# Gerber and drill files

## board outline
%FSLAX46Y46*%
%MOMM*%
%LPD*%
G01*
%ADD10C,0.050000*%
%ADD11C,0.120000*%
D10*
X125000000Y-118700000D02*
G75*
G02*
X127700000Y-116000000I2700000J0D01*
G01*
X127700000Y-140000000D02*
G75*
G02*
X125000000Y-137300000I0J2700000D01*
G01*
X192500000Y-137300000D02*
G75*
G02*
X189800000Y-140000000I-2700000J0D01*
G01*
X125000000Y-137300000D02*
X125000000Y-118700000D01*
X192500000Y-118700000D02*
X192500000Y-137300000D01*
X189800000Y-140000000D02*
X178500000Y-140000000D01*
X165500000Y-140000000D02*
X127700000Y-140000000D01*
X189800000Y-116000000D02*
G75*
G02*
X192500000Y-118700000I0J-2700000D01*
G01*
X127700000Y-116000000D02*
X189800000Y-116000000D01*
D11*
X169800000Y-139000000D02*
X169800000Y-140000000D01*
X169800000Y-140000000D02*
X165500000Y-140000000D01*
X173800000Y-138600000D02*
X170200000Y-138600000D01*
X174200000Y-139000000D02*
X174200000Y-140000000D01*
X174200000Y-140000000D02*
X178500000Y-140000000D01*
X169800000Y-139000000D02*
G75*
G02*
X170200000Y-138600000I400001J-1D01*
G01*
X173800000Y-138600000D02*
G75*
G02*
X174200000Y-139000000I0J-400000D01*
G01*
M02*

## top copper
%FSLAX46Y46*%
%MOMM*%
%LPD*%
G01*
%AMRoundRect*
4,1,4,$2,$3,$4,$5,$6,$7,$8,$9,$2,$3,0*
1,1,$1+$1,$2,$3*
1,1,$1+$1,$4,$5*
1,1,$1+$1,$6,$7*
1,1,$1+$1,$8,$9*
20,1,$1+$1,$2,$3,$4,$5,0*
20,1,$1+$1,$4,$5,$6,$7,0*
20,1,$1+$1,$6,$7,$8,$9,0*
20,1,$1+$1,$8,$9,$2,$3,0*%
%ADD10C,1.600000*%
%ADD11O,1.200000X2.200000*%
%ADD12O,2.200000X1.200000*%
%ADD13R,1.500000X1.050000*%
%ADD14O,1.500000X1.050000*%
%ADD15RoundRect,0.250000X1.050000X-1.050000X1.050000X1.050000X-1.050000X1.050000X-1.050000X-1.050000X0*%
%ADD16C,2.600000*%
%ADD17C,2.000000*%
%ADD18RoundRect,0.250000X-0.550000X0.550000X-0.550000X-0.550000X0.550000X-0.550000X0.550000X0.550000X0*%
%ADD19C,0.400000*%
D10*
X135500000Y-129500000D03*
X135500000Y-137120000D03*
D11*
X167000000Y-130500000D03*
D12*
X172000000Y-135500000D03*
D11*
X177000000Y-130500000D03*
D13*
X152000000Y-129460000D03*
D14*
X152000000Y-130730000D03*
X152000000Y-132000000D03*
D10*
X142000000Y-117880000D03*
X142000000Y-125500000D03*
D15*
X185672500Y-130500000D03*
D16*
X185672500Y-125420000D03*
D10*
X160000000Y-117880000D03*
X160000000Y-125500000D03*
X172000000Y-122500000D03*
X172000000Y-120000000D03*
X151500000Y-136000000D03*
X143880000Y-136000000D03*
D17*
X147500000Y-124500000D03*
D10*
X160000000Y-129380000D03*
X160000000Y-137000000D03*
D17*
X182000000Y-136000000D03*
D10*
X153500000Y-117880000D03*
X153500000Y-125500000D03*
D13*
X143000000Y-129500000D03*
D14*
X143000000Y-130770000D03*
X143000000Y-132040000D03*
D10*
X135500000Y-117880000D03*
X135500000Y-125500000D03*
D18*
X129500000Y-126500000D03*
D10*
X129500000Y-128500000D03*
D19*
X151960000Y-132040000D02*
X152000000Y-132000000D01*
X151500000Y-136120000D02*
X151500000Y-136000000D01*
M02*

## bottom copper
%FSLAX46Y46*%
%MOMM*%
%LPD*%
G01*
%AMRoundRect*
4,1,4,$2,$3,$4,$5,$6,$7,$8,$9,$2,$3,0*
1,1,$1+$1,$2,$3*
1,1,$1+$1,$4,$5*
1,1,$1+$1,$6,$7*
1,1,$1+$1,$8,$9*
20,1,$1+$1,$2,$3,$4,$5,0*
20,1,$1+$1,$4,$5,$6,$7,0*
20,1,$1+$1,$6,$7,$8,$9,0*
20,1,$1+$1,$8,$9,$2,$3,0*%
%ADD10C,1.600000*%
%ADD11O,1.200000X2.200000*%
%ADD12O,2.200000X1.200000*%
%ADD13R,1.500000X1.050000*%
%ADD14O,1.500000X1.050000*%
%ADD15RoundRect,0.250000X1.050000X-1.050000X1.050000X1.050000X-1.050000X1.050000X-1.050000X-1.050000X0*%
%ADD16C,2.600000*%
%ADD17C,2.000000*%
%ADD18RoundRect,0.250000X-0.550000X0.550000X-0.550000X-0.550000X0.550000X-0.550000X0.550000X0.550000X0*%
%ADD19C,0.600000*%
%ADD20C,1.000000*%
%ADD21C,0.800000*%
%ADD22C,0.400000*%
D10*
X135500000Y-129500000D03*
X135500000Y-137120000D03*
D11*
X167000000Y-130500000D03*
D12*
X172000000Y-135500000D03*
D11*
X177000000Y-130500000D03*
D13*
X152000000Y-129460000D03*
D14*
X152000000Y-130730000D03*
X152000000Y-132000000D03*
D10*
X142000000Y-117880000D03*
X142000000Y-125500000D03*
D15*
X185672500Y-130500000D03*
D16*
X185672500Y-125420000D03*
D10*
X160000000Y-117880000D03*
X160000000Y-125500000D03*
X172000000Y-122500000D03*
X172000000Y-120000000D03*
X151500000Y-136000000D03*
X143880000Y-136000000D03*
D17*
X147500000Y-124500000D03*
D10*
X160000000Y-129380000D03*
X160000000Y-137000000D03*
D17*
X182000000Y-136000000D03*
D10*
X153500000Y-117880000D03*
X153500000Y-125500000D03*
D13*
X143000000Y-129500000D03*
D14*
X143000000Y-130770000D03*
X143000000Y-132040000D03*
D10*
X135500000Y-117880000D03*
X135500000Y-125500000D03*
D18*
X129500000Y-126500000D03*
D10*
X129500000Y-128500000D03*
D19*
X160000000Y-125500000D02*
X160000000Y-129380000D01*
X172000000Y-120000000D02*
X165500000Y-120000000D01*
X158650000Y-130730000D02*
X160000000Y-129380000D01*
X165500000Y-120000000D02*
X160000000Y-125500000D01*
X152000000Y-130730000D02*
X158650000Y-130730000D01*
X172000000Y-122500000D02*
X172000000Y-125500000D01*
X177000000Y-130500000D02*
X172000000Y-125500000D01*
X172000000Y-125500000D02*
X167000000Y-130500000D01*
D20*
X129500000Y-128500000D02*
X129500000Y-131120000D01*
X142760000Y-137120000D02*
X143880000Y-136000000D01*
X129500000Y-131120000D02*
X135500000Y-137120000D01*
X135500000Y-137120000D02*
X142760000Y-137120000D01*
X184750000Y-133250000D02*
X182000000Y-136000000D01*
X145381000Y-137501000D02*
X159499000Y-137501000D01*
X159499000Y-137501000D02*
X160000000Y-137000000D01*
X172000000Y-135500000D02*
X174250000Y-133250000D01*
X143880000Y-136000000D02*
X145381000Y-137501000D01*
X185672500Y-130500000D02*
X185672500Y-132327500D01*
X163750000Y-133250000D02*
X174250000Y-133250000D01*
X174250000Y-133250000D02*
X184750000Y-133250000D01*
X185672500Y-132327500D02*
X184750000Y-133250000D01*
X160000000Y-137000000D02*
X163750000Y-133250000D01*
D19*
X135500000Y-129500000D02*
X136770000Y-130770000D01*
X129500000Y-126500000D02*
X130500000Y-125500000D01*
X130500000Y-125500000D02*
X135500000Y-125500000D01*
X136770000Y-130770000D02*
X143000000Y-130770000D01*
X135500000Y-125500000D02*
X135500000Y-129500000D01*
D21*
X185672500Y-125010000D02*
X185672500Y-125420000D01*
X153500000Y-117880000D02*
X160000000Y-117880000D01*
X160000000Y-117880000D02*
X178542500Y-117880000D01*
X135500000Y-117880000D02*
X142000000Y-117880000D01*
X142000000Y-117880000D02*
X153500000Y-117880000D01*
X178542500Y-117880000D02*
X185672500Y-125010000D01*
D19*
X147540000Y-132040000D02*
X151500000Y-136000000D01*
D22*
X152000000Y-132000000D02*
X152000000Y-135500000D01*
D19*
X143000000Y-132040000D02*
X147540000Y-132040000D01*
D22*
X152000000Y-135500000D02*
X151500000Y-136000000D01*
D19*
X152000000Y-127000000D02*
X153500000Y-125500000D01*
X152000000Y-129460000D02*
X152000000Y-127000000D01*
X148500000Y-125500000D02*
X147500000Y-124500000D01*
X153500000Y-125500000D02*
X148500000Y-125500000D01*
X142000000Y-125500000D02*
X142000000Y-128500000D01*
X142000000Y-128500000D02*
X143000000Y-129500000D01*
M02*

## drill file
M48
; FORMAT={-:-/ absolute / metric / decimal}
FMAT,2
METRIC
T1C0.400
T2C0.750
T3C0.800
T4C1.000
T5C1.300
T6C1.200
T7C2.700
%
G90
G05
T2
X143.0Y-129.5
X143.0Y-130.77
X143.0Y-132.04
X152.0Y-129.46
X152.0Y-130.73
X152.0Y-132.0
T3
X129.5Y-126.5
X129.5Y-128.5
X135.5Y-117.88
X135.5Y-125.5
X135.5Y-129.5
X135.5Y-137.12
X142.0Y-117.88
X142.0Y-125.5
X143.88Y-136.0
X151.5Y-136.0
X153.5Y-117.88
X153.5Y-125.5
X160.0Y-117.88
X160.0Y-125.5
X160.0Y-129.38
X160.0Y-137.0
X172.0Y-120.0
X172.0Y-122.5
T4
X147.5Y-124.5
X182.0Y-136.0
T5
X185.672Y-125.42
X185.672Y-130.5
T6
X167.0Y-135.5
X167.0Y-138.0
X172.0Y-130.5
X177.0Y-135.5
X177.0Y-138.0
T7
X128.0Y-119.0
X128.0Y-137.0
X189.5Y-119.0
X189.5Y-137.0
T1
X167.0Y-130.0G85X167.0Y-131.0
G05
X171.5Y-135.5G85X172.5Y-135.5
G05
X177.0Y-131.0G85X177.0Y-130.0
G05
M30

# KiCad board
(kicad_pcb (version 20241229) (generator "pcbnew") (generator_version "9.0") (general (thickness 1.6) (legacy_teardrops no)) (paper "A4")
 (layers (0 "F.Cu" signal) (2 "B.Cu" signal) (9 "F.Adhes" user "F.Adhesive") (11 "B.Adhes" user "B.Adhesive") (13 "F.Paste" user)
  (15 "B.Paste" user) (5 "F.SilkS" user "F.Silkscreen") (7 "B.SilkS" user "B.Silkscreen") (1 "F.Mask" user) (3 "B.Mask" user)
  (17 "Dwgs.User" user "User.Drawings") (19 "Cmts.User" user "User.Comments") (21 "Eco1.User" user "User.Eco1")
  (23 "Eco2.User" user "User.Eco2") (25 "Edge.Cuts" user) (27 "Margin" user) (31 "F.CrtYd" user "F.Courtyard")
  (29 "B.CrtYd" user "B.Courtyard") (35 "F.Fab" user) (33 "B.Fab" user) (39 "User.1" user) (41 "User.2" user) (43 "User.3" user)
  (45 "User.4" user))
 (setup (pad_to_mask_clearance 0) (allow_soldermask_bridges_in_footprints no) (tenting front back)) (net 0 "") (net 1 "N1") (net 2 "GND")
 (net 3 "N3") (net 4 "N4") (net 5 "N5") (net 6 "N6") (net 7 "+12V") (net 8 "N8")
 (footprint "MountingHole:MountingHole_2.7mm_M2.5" (layer "F.Cu") (at 128 137)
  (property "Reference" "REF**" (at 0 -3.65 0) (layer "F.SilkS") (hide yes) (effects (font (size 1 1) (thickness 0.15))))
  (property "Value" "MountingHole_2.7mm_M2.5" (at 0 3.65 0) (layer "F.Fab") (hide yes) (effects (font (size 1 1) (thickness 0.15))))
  (pad "" np_thru_hole circle (at 0 0) (size 2.7 2.7) (drill 2.7) (layers "*.Cu" "*.Mask")))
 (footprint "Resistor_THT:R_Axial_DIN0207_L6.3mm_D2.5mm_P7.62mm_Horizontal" (layer "F.Cu") (at 135.5 129.5 -90)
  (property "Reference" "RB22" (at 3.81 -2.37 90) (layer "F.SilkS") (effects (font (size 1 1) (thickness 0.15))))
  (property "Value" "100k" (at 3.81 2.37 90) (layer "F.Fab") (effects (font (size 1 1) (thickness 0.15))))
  (pad "1" thru_hole circle (at 0 0 270) (size 1.6 1.6) (drill 0.8) (layers "*.Cu" "*.Mask") (remove_unused_layers no) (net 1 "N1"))
  (pad "2" thru_hole circle (at 7.62 0 270) (size 1.6 1.6) (drill 0.8) (layers "*.Cu" "*.Mask") (remove_unused_layers no) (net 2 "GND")))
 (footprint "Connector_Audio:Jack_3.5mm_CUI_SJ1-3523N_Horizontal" (layer "F.Cu") (at 172 135.5)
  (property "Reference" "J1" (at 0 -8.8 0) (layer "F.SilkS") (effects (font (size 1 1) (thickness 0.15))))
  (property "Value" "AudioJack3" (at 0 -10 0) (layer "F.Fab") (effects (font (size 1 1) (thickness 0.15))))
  (fp_line (start -2.2 3.5) (end -2.2 4.5) (stroke (width 0.12) (type solid)) (layer "Edge.Cuts"))
  (fp_line (start -2.2 4.5) (end -6.5 4.5) (stroke (width 0.12) (type solid)) (layer "Edge.Cuts"))
  (fp_line (start 1.8 3.1) (end -1.8 3.1) (stroke (width 0.12) (type solid)) (layer "Edge.Cuts"))
  (fp_line (start 2.2 3.5) (end 2.2 4.5) (stroke (width 0.12) (type solid)) (layer "Edge.Cuts"))
  (fp_line (start 2.2 4.5) (end 6.5 4.5) (stroke (width 0.12) (type solid)) (layer "Edge.Cuts"))
  (fp_arc (start -2.2 3.5) (mid -2.082843 3.217158) (end -1.8 3.1) (stroke (width 0.12) (type solid)) (layer "Edge.Cuts"))
  (fp_arc (start 1.8 3.1) (mid 2.082843 3.217157) (end 2.2 3.5) (stroke (width 0.12) (type solid)) (layer "Edge.Cuts"))
  (pad "" np_thru_hole circle (at -5 0) (size 1.2 1.2) (drill 1.2) (layers "*.Cu" "*.Mask"))
  (pad "" np_thru_hole circle (at -5 2.5) (size 1.2 1.2) (drill 1.2) (layers "*.Cu" "*.Mask"))
  (pad "" np_thru_hole circle (at 0 -5) (size 1.2 1.2) (drill 1.2) (layers "*.Cu" "*.Mask"))
  (pad "" np_thru_hole circle (at 5 0) (size 1.2 1.2) (drill 1.2) (layers "*.Cu" "*.Mask"))
  (pad "" np_thru_hole circle (at 5 2.5) (size 1.2 1.2) (drill 1.2) (layers "*.Cu" "*.Mask"))
  (pad "R" thru_hole oval (at -5 -5) (size 1.2 2.2) (drill oval 0.4 1.4) (layers "*.Cu" "*.Mask") (remove_unused_layers no) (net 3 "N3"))
  (pad "S" thru_hole oval (at 0 0) (size 2.2 1.2) (drill oval 1.4 0.4) (layers "*.Cu" "*.Mask") (remove_unused_layers no) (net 2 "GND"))
  (pad "T" thru_hole oval (at 5 -5 180) (size 1.2 2.2) (drill oval 0.4 1.4) (layers "*.Cu" "*.Mask") (remove_unused_layers no) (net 3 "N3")))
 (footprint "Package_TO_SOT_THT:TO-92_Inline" (layer "F.Cu") (at 152 129.46 -90)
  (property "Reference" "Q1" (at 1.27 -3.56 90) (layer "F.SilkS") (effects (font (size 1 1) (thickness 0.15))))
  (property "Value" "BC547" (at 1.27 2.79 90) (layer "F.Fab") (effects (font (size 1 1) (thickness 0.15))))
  (pad "1" thru_hole rect (at 0 0 270) (size 1.05 1.5) (drill 0.75) (layers "*.Cu" "*.Mask") (remove_unused_layers no) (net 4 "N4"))
  (pad "2" thru_hole oval (at 1.27 0 270) (size 1.05 1.5) (drill 0.75) (layers "*.Cu" "*.Mask") (remove_unused_layers no) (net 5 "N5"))
  (pad "3" thru_hole oval (at 2.54 0 270) (size 1.05 1.5) (drill 0.75) (layers "*.Cu" "*.Mask") (remove_unused_layers no) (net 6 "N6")))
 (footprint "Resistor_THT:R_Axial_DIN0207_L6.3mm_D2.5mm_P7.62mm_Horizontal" (layer "F.Cu") (at 142 117.88 -90)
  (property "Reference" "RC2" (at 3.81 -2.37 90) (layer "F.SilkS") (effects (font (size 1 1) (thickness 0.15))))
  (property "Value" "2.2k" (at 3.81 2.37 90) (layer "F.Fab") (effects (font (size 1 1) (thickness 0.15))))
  (pad "1" thru_hole circle (at 0 0 270) (size 1.6 1.6) (drill 0.8) (layers "*.Cu" "*.Mask") (remove_unused_layers no) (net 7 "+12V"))
  (pad "2" thru_hole circle (at 7.62 0 270) (size 1.6 1.6) (drill 0.8) (layers "*.Cu" "*.Mask") (remove_unused_layers no) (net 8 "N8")))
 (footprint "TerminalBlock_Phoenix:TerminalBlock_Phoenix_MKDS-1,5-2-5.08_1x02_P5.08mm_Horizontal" (layer "F.Cu") (at 185.6725 130.5 90)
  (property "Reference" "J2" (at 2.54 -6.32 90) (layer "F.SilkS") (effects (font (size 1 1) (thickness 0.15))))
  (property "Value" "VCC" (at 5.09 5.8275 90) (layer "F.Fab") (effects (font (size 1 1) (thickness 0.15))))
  (pad "1" thru_hole roundrect (at 0 0 90) (size 2.6 2.6) (drill 1.3) (layers "*.Cu" "*.Mask") (remove_unused_layers no)
   (roundrect_rratio 0.096154) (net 2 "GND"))
  (pad "2" thru_hole circle (at 5.08 0 90) (size 2.6 2.6) (drill 1.3) (layers "*.Cu" "*.Mask") (remove_unused_layers no) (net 7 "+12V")))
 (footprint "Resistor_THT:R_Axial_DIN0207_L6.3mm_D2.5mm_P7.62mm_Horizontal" (layer "F.Cu") (at 160 117.88 -90)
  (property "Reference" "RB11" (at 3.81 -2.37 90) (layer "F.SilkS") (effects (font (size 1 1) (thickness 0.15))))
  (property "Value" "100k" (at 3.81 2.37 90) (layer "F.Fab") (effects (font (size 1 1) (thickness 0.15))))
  (pad "1" thru_hole circle (at 0 0 270) (size 1.6 1.6) (drill 0.8) (layers "*.Cu" "*.Mask") (remove_unused_layers no) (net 7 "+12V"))
  (pad "2" thru_hole circle (at 7.62 0 270) (size 1.6 1.6) (drill 0.8) (layers "*.Cu" "*.Mask") (remove_unused_layers no) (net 5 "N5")))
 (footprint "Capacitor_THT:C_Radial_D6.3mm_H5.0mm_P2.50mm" (layer "F.Cu") (at 172 122.5 90)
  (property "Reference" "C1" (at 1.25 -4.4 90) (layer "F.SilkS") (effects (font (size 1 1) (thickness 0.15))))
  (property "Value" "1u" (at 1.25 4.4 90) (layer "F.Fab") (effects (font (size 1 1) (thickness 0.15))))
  (pad "1" thru_hole circle (at 0 0 90) (size 1.6 1.6) (drill 0.8) (layers "*.Cu" "*.Mask") (remove_unused_layers no) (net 3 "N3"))
  (pad "2" thru_hole circle (at 2.5 0 90) (size 1.6 1.6) (drill 0.8) (layers "*.Cu" "*.Mask") (remove_unused_layers no) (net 5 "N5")))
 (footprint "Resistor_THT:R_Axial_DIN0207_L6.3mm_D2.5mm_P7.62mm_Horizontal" (layer "F.Cu") (at 151.5 136 180)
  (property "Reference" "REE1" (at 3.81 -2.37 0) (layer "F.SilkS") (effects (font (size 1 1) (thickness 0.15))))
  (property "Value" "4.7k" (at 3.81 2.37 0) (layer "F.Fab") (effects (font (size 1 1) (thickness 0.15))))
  (pad "1" thru_hole circle (at 0 0 180) (size 1.6 1.6) (drill 0.8) (layers "*.Cu" "*.Mask") (remove_unused_layers no) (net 6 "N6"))
  (pad "2" thru_hole circle (at 7.62 0 180) (size 1.6 1.6) (drill 0.8) (layers "*.Cu" "*.Mask") (remove_unused_layers no) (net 2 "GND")))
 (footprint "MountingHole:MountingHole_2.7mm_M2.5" (layer "F.Cu") (at 189.5 137)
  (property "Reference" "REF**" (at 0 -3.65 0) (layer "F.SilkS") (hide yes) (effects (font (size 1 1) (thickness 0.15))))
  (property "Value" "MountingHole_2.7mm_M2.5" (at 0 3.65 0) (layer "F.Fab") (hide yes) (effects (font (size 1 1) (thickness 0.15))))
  (pad "" np_thru_hole circle (at 0 0) (size 2.7 2.7) (drill 2.7) (layers "*.Cu" "*.Mask")))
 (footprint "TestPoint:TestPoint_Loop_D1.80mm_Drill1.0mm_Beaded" (layer "F.Cu") (at 147.5 124.5)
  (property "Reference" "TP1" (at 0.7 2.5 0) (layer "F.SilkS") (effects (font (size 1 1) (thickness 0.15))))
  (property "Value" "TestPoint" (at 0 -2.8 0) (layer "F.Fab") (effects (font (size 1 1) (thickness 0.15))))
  (pad "1" thru_hole circle (at 0 0) (size 2 2) (drill 1) (layers "*.Cu" "*.Mask") (remove_unused_layers no) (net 4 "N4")))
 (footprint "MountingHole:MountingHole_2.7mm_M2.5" (layer "F.Cu") (at 189.5 119)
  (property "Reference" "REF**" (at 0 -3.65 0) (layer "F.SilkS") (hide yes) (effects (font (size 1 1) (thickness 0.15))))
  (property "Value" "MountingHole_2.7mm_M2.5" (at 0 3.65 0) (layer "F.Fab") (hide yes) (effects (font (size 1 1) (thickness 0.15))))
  (pad "" np_thru_hole circle (at 0 0) (size 2.7 2.7) (drill 2.7) (layers "*.Cu" "*.Mask")))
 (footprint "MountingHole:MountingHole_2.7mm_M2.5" (layer "F.Cu") (at 128 119)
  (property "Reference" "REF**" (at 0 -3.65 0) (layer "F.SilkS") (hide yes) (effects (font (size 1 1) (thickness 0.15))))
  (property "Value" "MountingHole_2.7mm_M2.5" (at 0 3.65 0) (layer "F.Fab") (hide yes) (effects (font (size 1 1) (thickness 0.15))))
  (pad "" np_thru_hole circle (at 0 0) (size 2.7 2.7) (drill 2.7) (layers "*.Cu" "*.Mask")))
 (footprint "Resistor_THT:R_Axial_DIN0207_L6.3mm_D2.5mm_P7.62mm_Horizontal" (layer "F.Cu") (at 160 129.38 -90)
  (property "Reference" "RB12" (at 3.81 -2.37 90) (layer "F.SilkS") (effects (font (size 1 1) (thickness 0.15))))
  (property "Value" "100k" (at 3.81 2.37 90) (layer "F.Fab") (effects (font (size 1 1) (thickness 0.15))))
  (pad "1" thru_hole circle (at 0 0 270) (size 1.6 1.6) (drill 0.8) (layers "*.Cu" "*.Mask") (remove_unused_layers no) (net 5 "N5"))
  (pad "2" thru_hole circle (at 7.62 0 270) (size 1.6 1.6) (drill 0.8) (layers "*.Cu" "*.Mask") (remove_unused_layers no) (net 2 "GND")))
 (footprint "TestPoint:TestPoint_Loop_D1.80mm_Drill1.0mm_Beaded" (layer "F.Cu") (at 182 136)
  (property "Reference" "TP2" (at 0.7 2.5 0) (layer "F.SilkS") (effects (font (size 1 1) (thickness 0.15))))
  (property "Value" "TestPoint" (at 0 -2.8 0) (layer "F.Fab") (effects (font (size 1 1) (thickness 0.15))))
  (pad "1" thru_hole circle (at 0 0) (size 2 2) (drill 1) (layers "*.Cu" "*.Mask") (remove_unused_layers no) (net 2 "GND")))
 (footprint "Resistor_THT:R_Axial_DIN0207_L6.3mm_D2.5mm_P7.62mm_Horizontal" (layer "F.Cu") (at 153.5 117.88 -90)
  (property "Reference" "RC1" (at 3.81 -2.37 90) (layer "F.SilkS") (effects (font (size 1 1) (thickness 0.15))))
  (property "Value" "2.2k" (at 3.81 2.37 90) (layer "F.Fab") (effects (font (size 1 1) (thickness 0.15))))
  (pad "1" thru_hole circle (at 0 0 270) (size 1.6 1.6) (drill 0.8) (layers "*.Cu" "*.Mask") (remove_unused_layers no) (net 7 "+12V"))
  (pad "2" thru_hole circle (at 7.62 0 270) (size 1.6 1.6) (drill 0.8) (layers "*.Cu" "*.Mask") (remove_unused_layers no) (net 4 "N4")))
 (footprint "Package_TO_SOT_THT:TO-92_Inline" (layer "F.Cu") (at 143 129.5 -90)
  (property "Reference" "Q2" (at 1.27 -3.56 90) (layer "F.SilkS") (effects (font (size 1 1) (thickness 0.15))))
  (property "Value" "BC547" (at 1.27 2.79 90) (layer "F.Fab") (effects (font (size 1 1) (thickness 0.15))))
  (pad "1" thru_hole rect (at 0 0 270) (size 1.05 1.5) (drill 0.75) (layers "*.Cu" "*.Mask") (remove_unused_layers no) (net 8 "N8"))
  (pad "2" thru_hole oval (at 1.27 0 270) (size 1.05 1.5) (drill 0.75) (layers "*.Cu" "*.Mask") (remove_unused_layers no) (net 1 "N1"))
  (pad "3" thru_hole oval (at 2.54 0 270) (size 1.05 1.5) (drill 0.75) (layers "*.Cu" "*.Mask") (remove_unused_layers no) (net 6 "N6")))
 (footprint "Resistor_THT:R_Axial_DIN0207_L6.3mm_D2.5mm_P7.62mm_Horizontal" (layer "F.Cu") (at 135.5 117.88 -90)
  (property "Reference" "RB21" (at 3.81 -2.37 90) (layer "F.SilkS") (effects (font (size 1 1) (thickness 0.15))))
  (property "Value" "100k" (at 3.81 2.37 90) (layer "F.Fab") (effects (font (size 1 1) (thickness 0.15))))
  (pad "1" thru_hole circle (at 0 0 270) (size 1.6 1.6) (drill 0.8) (layers "*.Cu" "*.Mask") (remove_unused_layers no) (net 7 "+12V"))
  (pad "2" thru_hole circle (at 7.62 0 270) (size 1.6 1.6) (drill 0.8) (layers "*.Cu" "*.Mask") (remove_unused_layers no) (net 1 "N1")))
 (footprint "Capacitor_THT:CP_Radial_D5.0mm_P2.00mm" (layer "F.Cu") (at 129.5 126.5 -90)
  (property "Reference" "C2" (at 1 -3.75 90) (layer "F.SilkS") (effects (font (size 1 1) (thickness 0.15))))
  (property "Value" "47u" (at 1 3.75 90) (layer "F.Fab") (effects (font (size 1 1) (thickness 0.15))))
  (pad "1" thru_hole roundrect (at 0 0 270) (size 1.6 1.6) (drill 0.8) (layers "*.Cu" "*.Mask") (remove_unused_layers no)
   (roundrect_rratio 0.15625) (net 1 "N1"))
  (pad "2" thru_hole circle (at 2 0 270) (size 1.6 1.6) (drill 0.8) (layers "*.Cu" "*.Mask") (remove_unused_layers no) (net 2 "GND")))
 (gr_arc (start 125 118.7) (mid 125.790812 116.790812) (end 127.7 116) (stroke (width 0.05) (type default)) (layer "Edge.Cuts"))
 (gr_arc (start 127.7 140) (mid 125.790812 139.209188) (end 125 137.3) (stroke (width 0.05) (type default)) (layer "Edge.Cuts"))
 (gr_arc (start 192.5 137.3) (mid 191.709188 139.209188) (end 189.8 140) (stroke (width 0.05) (type default)) (layer "Edge.Cuts"))
 (gr_line (start 125 137.3) (end 125 118.7) (stroke (width 0.05) (type default)) (layer "Edge.Cuts"))
 (gr_line (start 192.5 118.7) (end 192.5 137.3) (stroke (width 0.05) (type default)) (layer "Edge.Cuts"))
 (gr_line (start 189.8 140) (end 178.5 140) (stroke (width 0.05) (type default)) (layer "Edge.Cuts"))
 (gr_line (start 165.5 140) (end 127.7 140) (stroke (width 0.05) (type default)) (layer "Edge.Cuts"))
 (gr_arc (start 189.8 116) (mid 191.709188 116.790812) (end 192.5 118.7) (stroke (width 0.05) (type default)) (layer "Edge.Cuts"))
 (gr_line (start 127.7 116) (end 189.8 116) (stroke (width 0.05) (type default)) (layer "Edge.Cuts"))
 (segment (start 160 125.5) (end 160 129.38) (width 0.6) (layer "B.Cu") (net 5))
 (segment (start 172 120) (end 165.5 120) (width 0.6) (layer "B.Cu") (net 5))
 (segment (start 158.65 130.73) (end 160 129.38) (width 0.6) (layer "B.Cu") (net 5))
 (segment (start 165.5 120) (end 160 125.5) (width 0.6) (layer "B.Cu") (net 5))
 (segment (start 152 130.73) (end 158.65 130.73) (width 0.6) (layer "B.Cu") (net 5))
 (segment (start 172 122.5) (end 172 125.5) (width 0.6) (layer "B.Cu") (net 3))
 (segment (start 177 130.5) (end 172 125.5) (width 0.6) (layer "B.Cu") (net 3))
 (segment (start 172 125.5) (end 167 130.5) (width 0.6) (layer "B.Cu") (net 3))
 (segment (start 129.5 128.5) (end 129.5 131.12) (width 1) (layer "B.Cu") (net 2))
 (segment (start 142.76 137.12) (end 143.88 136) (width 1) (layer "B.Cu") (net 2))
 (segment (start 129.5 131.12) (end 135.5 137.12) (width 1) (layer "B.Cu") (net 2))
 (segment (start 135.5 137.12) (end 142.76 137.12) (width 1) (layer "B.Cu") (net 2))
 (segment (start 184.75 133.25) (end 182 136) (width 1) (layer "B.Cu") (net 2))
 (segment (start 145.381 137.501) (end 159.499 137.501) (width 1) (layer "B.Cu") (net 2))
 (segment (start 159.499 137.501) (end 160 137) (width 1) (layer "B.Cu") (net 2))
 (segment (start 172 135.5) (end 174.25 133.25) (width 1) (layer "B.Cu") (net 2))
 (segment (start 143.88 136) (end 145.381 137.501) (width 1) (layer "B.Cu") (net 2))
 (segment (start 185.6725 130.5) (end 185.6725 132.3275) (width 1) (layer "B.Cu") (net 2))
 (segment (start 163.75 133.25) (end 174.25 133.25) (width 1) (layer "B.Cu") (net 2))
 (segment (start 174.25 133.25) (end 184.75 133.25) (width 1) (layer "B.Cu") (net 2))
 (segment (start 185.6725 132.3275) (end 184.75 133.25) (width 1) (layer "B.Cu") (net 2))
 (segment (start 160 137) (end 163.75 133.25) (width 1) (layer "B.Cu") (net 2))
 (segment (start 135.5 129.5) (end 136.77 130.77) (width 0.6) (layer "B.Cu") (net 1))
 (segment (start 129.5 126.5) (end 130.5 125.5) (width 0.6) (layer "B.Cu") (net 1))
 (segment (start 130.5 125.5) (end 135.5 125.5) (width 0.6) (layer "B.Cu") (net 1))
 (segment (start 136.77 130.77) (end 143 130.77) (width 0.6) (layer "B.Cu") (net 1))
 (segment (start 135.5 125.5) (end 135.5 129.5) (width 0.6) (layer "B.Cu") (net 1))
 (segment (start 185.6725 125.01) (end 185.6725 125.42) (width 0.8) (layer "B.Cu") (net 7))
 (segment (start 153.5 117.88) (end 160 117.88) (width 0.8) (layer "B.Cu") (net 7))
 (segment (start 160 117.88) (end 178.5425 117.88) (width 0.8) (layer "B.Cu") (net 7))
 (segment (start 135.5 117.88) (end 142 117.88) (width 0.8) (layer "B.Cu") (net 7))
 (segment (start 142 117.88) (end 153.5 117.88) (width 0.8) (layer "B.Cu") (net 7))
 (segment (start 178.5425 117.88) (end 185.6725 125.01) (width 0.8) (layer "B.Cu") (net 7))
 (segment (start 151.96 132.04) (end 152 132) (width 0.4) (layer "F.Cu") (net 6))
 (segment (start 151.5 136.12) (end 151.5 136) (width 0.4) (layer "F.Cu") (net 6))
 (segment (start 147.54 132.04) (end 151.5 136) (width 0.6) (layer "B.Cu") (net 6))
 (segment (start 152 132) (end 152 135.5) (width 0.4) (layer "B.Cu") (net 6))
 (segment (start 143 132.04) (end 147.54 132.04) (width 0.6) (layer "B.Cu") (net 6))
 (segment (start 152 135.5) (end 151.5 136) (width 0.4) (layer "B.Cu") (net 6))
 (segment (start 152 127) (end 153.5 125.5) (width 0.6) (layer "B.Cu") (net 4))
 (segment (start 152 129.46) (end 152 127) (width 0.6) (layer "B.Cu") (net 4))
 (segment (start 148.5 125.5) (end 147.5 124.5) (width 0.6) (layer "B.Cu") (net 4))
 (segment (start 153.5 125.5) (end 148.5 125.5) (width 0.6) (layer "B.Cu") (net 4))
 (segment (start 142 125.5) (end 142 128.5) (width 0.6) (layer "B.Cu") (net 8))
 (segment (start 142 128.5) (end 143 129.5) (width 0.6) (layer "B.Cu") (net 8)))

